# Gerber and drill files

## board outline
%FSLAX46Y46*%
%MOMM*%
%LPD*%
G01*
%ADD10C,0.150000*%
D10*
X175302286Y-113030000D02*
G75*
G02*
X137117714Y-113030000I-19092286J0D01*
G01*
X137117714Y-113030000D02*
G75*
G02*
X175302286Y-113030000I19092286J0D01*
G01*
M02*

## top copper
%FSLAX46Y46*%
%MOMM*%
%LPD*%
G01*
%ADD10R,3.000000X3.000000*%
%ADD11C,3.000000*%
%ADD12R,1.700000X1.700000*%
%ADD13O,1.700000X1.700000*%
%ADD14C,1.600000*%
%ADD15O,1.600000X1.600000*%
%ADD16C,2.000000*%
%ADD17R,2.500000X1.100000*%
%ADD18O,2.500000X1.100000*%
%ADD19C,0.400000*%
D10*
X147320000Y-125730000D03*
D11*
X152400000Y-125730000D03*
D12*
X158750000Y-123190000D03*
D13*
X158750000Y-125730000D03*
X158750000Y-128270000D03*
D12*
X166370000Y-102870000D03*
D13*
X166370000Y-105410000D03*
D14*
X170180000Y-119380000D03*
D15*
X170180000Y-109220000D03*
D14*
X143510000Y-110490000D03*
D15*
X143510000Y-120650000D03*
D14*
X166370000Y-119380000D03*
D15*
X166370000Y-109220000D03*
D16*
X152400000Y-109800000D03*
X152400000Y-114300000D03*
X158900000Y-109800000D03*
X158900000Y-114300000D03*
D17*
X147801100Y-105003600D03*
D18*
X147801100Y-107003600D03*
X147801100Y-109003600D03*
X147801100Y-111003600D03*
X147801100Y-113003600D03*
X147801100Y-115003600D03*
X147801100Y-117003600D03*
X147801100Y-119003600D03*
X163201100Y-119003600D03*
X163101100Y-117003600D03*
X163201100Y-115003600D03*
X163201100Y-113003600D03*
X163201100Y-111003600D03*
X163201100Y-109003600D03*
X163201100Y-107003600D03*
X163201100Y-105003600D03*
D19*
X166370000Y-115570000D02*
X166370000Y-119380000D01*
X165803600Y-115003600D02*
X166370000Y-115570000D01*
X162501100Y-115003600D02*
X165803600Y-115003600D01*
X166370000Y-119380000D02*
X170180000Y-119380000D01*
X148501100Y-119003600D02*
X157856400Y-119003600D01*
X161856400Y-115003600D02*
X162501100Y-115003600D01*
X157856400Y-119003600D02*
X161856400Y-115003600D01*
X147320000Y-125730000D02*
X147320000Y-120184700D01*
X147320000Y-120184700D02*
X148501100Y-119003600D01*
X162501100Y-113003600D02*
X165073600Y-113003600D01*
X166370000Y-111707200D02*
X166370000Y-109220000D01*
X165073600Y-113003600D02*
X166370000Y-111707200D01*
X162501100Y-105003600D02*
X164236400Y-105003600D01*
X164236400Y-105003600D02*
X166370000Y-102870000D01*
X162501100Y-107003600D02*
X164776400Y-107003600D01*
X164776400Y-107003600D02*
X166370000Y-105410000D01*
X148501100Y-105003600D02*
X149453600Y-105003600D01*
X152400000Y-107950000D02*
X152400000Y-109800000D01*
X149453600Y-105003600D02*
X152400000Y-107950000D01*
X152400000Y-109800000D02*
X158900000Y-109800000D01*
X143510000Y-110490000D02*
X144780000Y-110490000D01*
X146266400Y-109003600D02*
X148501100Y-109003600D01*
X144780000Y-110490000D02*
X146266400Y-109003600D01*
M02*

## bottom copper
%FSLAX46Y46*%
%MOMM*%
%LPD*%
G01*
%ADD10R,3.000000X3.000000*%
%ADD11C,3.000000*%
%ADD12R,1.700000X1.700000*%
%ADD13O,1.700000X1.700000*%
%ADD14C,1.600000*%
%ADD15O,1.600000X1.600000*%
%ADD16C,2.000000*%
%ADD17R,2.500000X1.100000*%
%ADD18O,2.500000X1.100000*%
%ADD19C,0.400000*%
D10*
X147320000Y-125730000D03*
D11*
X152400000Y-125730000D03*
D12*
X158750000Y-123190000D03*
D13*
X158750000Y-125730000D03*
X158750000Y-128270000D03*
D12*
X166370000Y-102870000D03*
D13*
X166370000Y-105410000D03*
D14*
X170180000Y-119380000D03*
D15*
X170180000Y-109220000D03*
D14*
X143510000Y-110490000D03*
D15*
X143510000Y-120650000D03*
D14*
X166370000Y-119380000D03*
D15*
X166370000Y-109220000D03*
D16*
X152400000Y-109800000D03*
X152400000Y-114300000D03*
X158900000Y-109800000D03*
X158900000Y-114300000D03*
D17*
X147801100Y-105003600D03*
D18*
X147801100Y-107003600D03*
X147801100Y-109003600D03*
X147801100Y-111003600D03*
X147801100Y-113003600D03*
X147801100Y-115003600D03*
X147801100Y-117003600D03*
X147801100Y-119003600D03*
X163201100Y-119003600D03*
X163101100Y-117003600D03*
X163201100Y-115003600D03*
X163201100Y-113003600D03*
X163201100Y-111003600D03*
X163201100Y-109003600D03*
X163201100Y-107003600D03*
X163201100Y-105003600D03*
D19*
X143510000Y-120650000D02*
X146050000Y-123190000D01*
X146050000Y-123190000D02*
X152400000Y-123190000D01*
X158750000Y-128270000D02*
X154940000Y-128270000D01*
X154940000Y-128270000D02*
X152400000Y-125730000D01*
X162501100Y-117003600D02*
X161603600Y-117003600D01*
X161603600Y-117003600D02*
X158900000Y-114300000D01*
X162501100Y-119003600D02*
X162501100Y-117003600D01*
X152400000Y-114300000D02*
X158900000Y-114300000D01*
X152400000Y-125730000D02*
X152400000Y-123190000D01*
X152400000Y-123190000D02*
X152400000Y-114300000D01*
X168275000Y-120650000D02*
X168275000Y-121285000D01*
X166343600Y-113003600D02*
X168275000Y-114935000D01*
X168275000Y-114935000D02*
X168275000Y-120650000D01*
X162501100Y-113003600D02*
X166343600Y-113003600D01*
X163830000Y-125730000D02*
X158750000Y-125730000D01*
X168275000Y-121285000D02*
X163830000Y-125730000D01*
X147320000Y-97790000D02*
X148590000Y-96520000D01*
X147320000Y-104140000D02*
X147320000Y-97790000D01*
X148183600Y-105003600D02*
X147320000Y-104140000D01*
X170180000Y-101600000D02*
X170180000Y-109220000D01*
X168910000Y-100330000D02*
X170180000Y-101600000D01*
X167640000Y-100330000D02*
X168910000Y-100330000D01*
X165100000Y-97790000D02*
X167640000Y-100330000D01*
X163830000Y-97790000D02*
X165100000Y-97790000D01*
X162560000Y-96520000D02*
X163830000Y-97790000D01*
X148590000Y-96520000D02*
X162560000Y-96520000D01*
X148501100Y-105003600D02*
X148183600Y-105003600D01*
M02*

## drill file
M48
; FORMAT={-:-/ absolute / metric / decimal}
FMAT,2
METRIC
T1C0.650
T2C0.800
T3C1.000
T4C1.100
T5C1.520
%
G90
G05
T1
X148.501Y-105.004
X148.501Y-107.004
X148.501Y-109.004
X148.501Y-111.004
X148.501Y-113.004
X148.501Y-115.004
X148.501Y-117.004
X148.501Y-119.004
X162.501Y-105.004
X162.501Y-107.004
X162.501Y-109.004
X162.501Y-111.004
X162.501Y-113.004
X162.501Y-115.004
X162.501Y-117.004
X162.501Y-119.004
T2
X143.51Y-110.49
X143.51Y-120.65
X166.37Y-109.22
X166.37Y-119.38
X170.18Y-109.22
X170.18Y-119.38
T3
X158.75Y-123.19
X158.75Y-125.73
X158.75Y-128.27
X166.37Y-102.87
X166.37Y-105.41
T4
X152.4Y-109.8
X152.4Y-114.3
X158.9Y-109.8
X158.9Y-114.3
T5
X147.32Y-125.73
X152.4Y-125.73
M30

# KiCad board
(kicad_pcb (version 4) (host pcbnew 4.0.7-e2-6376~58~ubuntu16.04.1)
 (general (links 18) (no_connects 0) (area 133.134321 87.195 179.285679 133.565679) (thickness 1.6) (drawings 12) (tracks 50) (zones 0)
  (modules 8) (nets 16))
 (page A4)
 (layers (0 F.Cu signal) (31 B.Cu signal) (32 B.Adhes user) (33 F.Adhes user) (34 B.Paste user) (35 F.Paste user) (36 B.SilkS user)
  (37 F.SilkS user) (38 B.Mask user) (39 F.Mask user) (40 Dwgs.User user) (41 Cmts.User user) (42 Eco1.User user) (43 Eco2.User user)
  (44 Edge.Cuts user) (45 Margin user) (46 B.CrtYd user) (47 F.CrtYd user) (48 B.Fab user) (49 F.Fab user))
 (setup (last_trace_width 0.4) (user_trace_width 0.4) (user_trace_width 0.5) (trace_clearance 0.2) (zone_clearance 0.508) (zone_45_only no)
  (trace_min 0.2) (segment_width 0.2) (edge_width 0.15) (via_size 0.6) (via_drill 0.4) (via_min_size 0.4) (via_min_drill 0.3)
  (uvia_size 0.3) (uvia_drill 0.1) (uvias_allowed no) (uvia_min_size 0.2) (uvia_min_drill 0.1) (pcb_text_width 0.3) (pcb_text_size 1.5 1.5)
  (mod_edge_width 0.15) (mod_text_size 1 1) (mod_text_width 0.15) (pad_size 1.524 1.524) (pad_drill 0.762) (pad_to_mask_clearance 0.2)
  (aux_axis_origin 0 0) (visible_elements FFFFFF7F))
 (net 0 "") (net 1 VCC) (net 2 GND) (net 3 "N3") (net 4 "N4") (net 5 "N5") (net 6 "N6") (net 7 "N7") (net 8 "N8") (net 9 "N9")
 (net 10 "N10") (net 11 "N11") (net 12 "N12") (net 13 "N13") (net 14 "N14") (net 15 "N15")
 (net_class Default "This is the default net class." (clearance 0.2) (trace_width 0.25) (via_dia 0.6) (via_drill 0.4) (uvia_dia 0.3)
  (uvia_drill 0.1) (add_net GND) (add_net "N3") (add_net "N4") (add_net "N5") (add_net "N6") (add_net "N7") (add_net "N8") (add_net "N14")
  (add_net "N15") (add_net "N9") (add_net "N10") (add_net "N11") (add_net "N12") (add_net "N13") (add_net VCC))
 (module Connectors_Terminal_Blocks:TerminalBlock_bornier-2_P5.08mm (layer F.Cu) (at 147.32 125.73)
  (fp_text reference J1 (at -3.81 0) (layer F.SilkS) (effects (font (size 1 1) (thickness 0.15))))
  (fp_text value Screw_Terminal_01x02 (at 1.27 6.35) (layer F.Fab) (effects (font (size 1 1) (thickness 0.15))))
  (pad 1 thru_hole rect (at 0 0) (size 3 3) (drill 1.52) (layers *.Cu *.Mask) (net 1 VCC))
  (pad 2 thru_hole circle (at 5.08 0) (size 3 3) (drill 1.52) (layers *.Cu *.Mask) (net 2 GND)))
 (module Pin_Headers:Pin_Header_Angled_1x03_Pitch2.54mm (layer F.Cu) (at 158.75 123.19)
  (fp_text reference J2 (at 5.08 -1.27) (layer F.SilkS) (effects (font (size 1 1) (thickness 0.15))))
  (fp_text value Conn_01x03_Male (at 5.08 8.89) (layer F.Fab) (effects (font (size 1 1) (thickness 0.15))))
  (pad 1 thru_hole rect (at 0 0) (size 1.7 1.7) (drill 1) (layers *.Cu *.Mask) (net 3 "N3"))
  (pad 2 thru_hole oval (at 0 2.54) (size 1.7 1.7) (drill 1) (layers *.Cu *.Mask) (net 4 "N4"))
  (pad 3 thru_hole oval (at 0 5.08) (size 1.7 1.7) (drill 1) (layers *.Cu *.Mask) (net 2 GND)))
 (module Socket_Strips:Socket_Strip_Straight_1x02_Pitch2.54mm (layer F.Cu) (at 166.37 102.87)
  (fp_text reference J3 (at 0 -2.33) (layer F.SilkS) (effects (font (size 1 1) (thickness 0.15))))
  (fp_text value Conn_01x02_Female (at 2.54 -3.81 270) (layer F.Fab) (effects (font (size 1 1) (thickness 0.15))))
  (pad 1 thru_hole rect (at 0 0) (size 1.7 1.7) (drill 1) (layers *.Cu *.Mask) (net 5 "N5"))
  (pad 2 thru_hole oval (at 0 2.54) (size 1.7 1.7) (drill 1) (layers *.Cu *.Mask) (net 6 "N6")))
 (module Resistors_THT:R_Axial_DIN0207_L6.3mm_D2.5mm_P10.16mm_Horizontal (layer F.Cu) (at 170.18 119.38 90)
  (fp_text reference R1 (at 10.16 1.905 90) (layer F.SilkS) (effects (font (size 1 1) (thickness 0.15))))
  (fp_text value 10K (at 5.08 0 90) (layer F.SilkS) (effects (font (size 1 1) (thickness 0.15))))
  (pad 1 thru_hole circle (at 0 0 90) (size 1.6 1.6) (drill 0.8) (layers *.Cu *.Mask) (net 1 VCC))
  (pad 2 thru_hole oval (at 10.16 0 90) (size 1.6 1.6) (drill 0.8) (layers *.Cu *.Mask) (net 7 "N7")))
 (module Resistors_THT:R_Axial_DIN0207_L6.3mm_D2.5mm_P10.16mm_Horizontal (layer F.Cu) (at 143.51 110.49 270)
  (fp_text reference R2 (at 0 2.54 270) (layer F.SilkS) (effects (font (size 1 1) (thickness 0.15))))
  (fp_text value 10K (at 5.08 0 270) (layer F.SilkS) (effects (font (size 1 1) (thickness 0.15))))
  (pad 1 thru_hole circle (at 0 0 270) (size 1.6 1.6) (drill 0.8) (layers *.Cu *.Mask) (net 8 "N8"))
  (pad 2 thru_hole oval (at 10.16 0 270) (size 1.6 1.6) (drill 0.8) (layers *.Cu *.Mask) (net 2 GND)))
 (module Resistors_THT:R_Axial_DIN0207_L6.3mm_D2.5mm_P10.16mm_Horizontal (layer F.Cu) (at 166.37 119.38 90)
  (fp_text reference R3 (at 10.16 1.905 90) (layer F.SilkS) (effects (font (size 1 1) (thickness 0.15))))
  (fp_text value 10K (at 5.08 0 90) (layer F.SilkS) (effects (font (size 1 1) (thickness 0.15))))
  (pad 1 thru_hole circle (at 0 0 90) (size 1.6 1.6) (drill 0.8) (layers *.Cu *.Mask) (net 1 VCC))
  (pad 2 thru_hole oval (at 10.16 0 90) (size 1.6 1.6) (drill 0.8) (layers *.Cu *.Mask) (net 4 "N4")))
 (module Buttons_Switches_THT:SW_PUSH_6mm (layer B.Cu) (at 152.4 114.3)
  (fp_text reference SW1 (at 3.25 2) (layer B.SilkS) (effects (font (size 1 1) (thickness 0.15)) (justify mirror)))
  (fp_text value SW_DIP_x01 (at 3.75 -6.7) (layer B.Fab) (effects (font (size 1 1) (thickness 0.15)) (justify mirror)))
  (pad 2 thru_hole circle (at 0 -4.5 270) (size 2 2) (drill 1.1) (layers *.Cu *.Mask) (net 7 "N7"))
  (pad 1 thru_hole circle (at 0 0 270) (size 2 2) (drill 1.1) (layers *.Cu *.Mask) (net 2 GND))
  (pad 2 thru_hole circle (at 6.5 -4.5 270) (size 2 2) (drill 1.1) (layers *.Cu *.Mask) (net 7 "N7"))
  (pad 1 thru_hole circle (at 6.5 0 270) (size 2 2) (drill 1.1) (layers *.Cu *.Mask) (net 2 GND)))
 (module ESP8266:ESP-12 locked (layer F.Cu) (at 148.5011 105.0036)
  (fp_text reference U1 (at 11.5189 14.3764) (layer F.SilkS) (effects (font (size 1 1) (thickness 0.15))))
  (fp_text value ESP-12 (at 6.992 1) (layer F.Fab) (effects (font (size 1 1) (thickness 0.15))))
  (pad 1 thru_hole rect (at 0 0) (size 2.5 1.1) (drill 0.65 (offset -0.7 0)) (layers *.Cu *.Mask F.SilkS) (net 7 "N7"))
  (pad 2 thru_hole oval (at 0 2) (size 2.5 1.1) (drill 0.65 (offset -0.7 0)) (layers *.Cu *.Mask F.SilkS) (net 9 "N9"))
  (pad 3 thru_hole oval (at 0 4) (size 2.5 1.1) (drill 0.65 (offset -0.7 0)) (layers *.Cu *.Mask F.SilkS) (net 8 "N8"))
  (pad 4 thru_hole oval (at 0 6) (size 2.5 1.1) (drill 0.65 (offset -0.7 0)) (layers *.Cu *.Mask F.SilkS) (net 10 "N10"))
  (pad 5 thru_hole oval (at 0 8) (size 2.5 1.1) (drill 0.65 (offset -0.7 0)) (layers *.Cu *.Mask F.SilkS) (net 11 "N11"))
  (pad 6 thru_hole oval (at 0 10) (size 2.5 1.1) (drill 0.65 (offset -0.7 0)) (layers *.Cu *.Mask F.SilkS) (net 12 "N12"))
  (pad 7 thru_hole oval (at 0 12) (size 2.5 1.1) (drill 0.65 (offset -0.7 0)) (layers *.Cu *.Mask F.SilkS) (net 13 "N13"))
  (pad 8 thru_hole oval (at 0 14) (size 2.5 1.1) (drill 0.65 (offset -0.7 0)) (layers *.Cu *.Mask F.SilkS) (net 1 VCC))
  (pad 9 thru_hole oval (at 14 14) (size 2.5 1.1) (drill 0.65 (offset 0.7 0)) (layers *.Cu *.Mask F.SilkS) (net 2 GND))
  (pad 10 thru_hole oval (at 14 12) (size 2.5 1.1) (drill 0.65 (offset 0.6 0)) (layers *.Cu *.Mask F.SilkS) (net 2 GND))
  (pad 11 thru_hole oval (at 14 10) (size 2.5 1.1) (drill 0.65 (offset 0.7 0)) (layers *.Cu *.Mask F.SilkS) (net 1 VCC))
  (pad 12 thru_hole oval (at 14 8) (size 2.5 1.1) (drill 0.65 (offset 0.7 0)) (layers *.Cu *.Mask F.SilkS) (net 4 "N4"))
  (pad 13 thru_hole oval (at 14 6) (size 2.5 1.1) (drill 0.65 (offset 0.7 0)) (layers *.Cu *.Mask F.SilkS) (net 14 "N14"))
  (pad 14 thru_hole oval (at 14 4) (size 2.5 1.1) (drill 0.65 (offset 0.7 0)) (layers *.Cu *.Mask F.SilkS) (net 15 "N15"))
  (pad 15 thru_hole oval (at 14 2) (size 2.5 1.1) (drill 0.65 (offset 0.7 0)) (layers *.Cu *.Mask F.SilkS) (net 6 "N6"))
  (pad 16 thru_hole oval (at 14 0) (size 2.5 1.1) (drill 0.65 (offset 0.7 0)) (layers *.Cu *.Mask F.SilkS) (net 5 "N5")))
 (gr_circle (center 156.21 113.03) (end 157.48 93.98) (layer Edge.Cuts) (width 0.15))
 (segment (start 166.37 115.57) (end 166.37 119.38) (width 0.4) (layer F.Cu) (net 1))
 (segment (start 165.8036 115.0036) (end 166.37 115.57) (width 0.4) (layer F.Cu) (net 1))
 (segment (start 162.5011 115.0036) (end 165.8036 115.0036) (width 0.4) (layer F.Cu) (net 1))
 (segment (start 166.37 119.38) (end 170.18 119.38) (width 0.4) (layer F.Cu) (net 1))
 (segment (start 148.5011 119.0036) (end 157.8564 119.0036) (width 0.4) (layer F.Cu) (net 1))
 (segment (start 161.8564 115.0036) (end 162.5011 115.0036) (width 0.4) (layer F.Cu) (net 1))
 (segment (start 157.8564 119.0036) (end 161.8564 115.0036) (width 0.4) (layer F.Cu) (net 1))
 (segment (start 147.32 125.73) (end 147.32 120.1847) (width 0.4) (layer F.Cu) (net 1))
 (segment (start 147.32 120.1847) (end 148.5011 119.0036) (width 0.4) (layer F.Cu) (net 1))
 (segment (start 143.51 120.65) (end 146.05 123.19) (width 0.4) (layer B.Cu) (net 2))
 (segment (start 146.05 123.19) (end 152.4 123.19) (width 0.4) (layer B.Cu) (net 2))
 (segment (start 158.75 128.27) (end 154.94 128.27) (width 0.4) (layer B.Cu) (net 2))
 (segment (start 154.94 128.27) (end 152.4 125.73) (width 0.4) (layer B.Cu) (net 2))
 (segment (start 162.5011 117.0036) (end 161.6036 117.0036) (width 0.4) (layer B.Cu) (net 2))
 (segment (start 161.6036 117.0036) (end 158.9 114.3) (width 0.4) (layer B.Cu) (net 2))
 (segment (start 162.5011 119.0036) (end 162.5011 117.0036) (width 0.4) (layer B.Cu) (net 2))
 (segment (start 152.4 114.3) (end 158.9 114.3) (width 0.4) (layer B.Cu) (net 2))
 (segment (start 152.4 125.73) (end 152.4 123.19) (width 0.4) (layer B.Cu) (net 2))
 (segment (start 152.4 123.19) (end 152.4 114.3) (width 0.4) (layer B.Cu) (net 2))
 (segment (start 168.275 120.65) (end 168.275 121.285) (width 0.4) (layer B.Cu) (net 4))
 (segment (start 166.3436 113.0036) (end 168.275 114.935) (width 0.4) (layer B.Cu) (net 4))
 (segment (start 168.275 114.935) (end 168.275 120.65) (width 0.4) (layer B.Cu) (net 4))
 (segment (start 162.5011 113.0036) (end 166.3436 113.0036) (width 0.4) (layer B.Cu) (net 4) (status 400000))
 (segment (start 163.83 125.73) (end 158.75 125.73) (width 0.4) (layer B.Cu) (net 4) (status 800000))
 (segment (start 168.275 121.285) (end 163.83 125.73) (width 0.4) (layer B.Cu) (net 4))
 (segment (start 162.5011 113.0036) (end 165.0736 113.0036) (width 0.4) (layer F.Cu) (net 4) (status 400000))
 (segment (start 166.37 111.7072) (end 166.37 109.22) (width 0.4) (layer F.Cu) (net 4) (status 800000))
 (segment (start 165.0736 113.0036) (end 166.37 111.7072) (width 0.4) (layer F.Cu) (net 4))
 (segment (start 162.5011 105.0036) (end 164.2364 105.0036) (width 0.4) (layer F.Cu) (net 5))
 (segment (start 164.2364 105.0036) (end 166.37 102.87) (width 0.4) (layer F.Cu) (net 5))
 (segment (start 162.5011 107.0036) (end 164.7764 107.0036) (width 0.4) (layer F.Cu) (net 6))
 (segment (start 164.7764 107.0036) (end 166.37 105.41) (width 0.4) (layer F.Cu) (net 6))
 (segment (start 147.32 97.79) (end 148.59 96.52) (width 0.4) (layer B.Cu) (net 7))
 (segment (start 147.32 104.14) (end 147.32 97.79) (width 0.4) (layer B.Cu) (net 7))
 (segment (start 148.1836 105.0036) (end 147.32 104.14) (width 0.4) (layer B.Cu) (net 7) (status 400000))
 (segment (start 170.18 101.6) (end 170.18 109.22) (width 0.4) (layer B.Cu) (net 7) (status 800000))
 (segment (start 168.91 100.33) (end 170.18 101.6) (width 0.4) (layer B.Cu) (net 7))
 (segment (start 167.64 100.33) (end 168.91 100.33) (width 0.4) (layer B.Cu) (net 7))
 (segment (start 165.1 97.79) (end 167.64 100.33) (width 0.4) (layer B.Cu) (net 7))
 (segment (start 163.83 97.79) (end 165.1 97.79) (width 0.4) (layer B.Cu) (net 7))
 (segment (start 162.56 96.52) (end 163.83 97.79) (width 0.4) (layer B.Cu) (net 7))
 (segment (start 148.59 96.52) (end 162.56 96.52) (width 0.4) (layer B.Cu) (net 7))
 (segment (start 148.5011 105.0036) (end 148.1836 105.0036) (width 0.4) (layer B.Cu) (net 7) (status C00000))
 (segment (start 148.5011 105.0036) (end 149.4536 105.0036) (width 0.4) (layer F.Cu) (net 7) (status 400000))
 (segment (start 152.4 107.95) (end 152.4 109.8) (width 0.4) (layer F.Cu) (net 7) (status 800000))
 (segment (start 149.4536 105.0036) (end 152.4 107.95) (width 0.4) (layer F.Cu) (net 7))
 (segment (start 152.4 109.8) (end 158.9 109.8) (width 0.4) (layer F.Cu) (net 7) (status C00000))
 (segment (start 143.51 110.49) (end 144.78 110.49) (width 0.4) (layer F.Cu) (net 8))
 (segment (start 146.2664 109.0036) (end 148.5011 109.0036) (width 0.4) (layer F.Cu) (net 8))
 (segment (start 144.78 110.49) (end 146.2664 109.0036) (width 0.4) (layer F.Cu) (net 8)))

